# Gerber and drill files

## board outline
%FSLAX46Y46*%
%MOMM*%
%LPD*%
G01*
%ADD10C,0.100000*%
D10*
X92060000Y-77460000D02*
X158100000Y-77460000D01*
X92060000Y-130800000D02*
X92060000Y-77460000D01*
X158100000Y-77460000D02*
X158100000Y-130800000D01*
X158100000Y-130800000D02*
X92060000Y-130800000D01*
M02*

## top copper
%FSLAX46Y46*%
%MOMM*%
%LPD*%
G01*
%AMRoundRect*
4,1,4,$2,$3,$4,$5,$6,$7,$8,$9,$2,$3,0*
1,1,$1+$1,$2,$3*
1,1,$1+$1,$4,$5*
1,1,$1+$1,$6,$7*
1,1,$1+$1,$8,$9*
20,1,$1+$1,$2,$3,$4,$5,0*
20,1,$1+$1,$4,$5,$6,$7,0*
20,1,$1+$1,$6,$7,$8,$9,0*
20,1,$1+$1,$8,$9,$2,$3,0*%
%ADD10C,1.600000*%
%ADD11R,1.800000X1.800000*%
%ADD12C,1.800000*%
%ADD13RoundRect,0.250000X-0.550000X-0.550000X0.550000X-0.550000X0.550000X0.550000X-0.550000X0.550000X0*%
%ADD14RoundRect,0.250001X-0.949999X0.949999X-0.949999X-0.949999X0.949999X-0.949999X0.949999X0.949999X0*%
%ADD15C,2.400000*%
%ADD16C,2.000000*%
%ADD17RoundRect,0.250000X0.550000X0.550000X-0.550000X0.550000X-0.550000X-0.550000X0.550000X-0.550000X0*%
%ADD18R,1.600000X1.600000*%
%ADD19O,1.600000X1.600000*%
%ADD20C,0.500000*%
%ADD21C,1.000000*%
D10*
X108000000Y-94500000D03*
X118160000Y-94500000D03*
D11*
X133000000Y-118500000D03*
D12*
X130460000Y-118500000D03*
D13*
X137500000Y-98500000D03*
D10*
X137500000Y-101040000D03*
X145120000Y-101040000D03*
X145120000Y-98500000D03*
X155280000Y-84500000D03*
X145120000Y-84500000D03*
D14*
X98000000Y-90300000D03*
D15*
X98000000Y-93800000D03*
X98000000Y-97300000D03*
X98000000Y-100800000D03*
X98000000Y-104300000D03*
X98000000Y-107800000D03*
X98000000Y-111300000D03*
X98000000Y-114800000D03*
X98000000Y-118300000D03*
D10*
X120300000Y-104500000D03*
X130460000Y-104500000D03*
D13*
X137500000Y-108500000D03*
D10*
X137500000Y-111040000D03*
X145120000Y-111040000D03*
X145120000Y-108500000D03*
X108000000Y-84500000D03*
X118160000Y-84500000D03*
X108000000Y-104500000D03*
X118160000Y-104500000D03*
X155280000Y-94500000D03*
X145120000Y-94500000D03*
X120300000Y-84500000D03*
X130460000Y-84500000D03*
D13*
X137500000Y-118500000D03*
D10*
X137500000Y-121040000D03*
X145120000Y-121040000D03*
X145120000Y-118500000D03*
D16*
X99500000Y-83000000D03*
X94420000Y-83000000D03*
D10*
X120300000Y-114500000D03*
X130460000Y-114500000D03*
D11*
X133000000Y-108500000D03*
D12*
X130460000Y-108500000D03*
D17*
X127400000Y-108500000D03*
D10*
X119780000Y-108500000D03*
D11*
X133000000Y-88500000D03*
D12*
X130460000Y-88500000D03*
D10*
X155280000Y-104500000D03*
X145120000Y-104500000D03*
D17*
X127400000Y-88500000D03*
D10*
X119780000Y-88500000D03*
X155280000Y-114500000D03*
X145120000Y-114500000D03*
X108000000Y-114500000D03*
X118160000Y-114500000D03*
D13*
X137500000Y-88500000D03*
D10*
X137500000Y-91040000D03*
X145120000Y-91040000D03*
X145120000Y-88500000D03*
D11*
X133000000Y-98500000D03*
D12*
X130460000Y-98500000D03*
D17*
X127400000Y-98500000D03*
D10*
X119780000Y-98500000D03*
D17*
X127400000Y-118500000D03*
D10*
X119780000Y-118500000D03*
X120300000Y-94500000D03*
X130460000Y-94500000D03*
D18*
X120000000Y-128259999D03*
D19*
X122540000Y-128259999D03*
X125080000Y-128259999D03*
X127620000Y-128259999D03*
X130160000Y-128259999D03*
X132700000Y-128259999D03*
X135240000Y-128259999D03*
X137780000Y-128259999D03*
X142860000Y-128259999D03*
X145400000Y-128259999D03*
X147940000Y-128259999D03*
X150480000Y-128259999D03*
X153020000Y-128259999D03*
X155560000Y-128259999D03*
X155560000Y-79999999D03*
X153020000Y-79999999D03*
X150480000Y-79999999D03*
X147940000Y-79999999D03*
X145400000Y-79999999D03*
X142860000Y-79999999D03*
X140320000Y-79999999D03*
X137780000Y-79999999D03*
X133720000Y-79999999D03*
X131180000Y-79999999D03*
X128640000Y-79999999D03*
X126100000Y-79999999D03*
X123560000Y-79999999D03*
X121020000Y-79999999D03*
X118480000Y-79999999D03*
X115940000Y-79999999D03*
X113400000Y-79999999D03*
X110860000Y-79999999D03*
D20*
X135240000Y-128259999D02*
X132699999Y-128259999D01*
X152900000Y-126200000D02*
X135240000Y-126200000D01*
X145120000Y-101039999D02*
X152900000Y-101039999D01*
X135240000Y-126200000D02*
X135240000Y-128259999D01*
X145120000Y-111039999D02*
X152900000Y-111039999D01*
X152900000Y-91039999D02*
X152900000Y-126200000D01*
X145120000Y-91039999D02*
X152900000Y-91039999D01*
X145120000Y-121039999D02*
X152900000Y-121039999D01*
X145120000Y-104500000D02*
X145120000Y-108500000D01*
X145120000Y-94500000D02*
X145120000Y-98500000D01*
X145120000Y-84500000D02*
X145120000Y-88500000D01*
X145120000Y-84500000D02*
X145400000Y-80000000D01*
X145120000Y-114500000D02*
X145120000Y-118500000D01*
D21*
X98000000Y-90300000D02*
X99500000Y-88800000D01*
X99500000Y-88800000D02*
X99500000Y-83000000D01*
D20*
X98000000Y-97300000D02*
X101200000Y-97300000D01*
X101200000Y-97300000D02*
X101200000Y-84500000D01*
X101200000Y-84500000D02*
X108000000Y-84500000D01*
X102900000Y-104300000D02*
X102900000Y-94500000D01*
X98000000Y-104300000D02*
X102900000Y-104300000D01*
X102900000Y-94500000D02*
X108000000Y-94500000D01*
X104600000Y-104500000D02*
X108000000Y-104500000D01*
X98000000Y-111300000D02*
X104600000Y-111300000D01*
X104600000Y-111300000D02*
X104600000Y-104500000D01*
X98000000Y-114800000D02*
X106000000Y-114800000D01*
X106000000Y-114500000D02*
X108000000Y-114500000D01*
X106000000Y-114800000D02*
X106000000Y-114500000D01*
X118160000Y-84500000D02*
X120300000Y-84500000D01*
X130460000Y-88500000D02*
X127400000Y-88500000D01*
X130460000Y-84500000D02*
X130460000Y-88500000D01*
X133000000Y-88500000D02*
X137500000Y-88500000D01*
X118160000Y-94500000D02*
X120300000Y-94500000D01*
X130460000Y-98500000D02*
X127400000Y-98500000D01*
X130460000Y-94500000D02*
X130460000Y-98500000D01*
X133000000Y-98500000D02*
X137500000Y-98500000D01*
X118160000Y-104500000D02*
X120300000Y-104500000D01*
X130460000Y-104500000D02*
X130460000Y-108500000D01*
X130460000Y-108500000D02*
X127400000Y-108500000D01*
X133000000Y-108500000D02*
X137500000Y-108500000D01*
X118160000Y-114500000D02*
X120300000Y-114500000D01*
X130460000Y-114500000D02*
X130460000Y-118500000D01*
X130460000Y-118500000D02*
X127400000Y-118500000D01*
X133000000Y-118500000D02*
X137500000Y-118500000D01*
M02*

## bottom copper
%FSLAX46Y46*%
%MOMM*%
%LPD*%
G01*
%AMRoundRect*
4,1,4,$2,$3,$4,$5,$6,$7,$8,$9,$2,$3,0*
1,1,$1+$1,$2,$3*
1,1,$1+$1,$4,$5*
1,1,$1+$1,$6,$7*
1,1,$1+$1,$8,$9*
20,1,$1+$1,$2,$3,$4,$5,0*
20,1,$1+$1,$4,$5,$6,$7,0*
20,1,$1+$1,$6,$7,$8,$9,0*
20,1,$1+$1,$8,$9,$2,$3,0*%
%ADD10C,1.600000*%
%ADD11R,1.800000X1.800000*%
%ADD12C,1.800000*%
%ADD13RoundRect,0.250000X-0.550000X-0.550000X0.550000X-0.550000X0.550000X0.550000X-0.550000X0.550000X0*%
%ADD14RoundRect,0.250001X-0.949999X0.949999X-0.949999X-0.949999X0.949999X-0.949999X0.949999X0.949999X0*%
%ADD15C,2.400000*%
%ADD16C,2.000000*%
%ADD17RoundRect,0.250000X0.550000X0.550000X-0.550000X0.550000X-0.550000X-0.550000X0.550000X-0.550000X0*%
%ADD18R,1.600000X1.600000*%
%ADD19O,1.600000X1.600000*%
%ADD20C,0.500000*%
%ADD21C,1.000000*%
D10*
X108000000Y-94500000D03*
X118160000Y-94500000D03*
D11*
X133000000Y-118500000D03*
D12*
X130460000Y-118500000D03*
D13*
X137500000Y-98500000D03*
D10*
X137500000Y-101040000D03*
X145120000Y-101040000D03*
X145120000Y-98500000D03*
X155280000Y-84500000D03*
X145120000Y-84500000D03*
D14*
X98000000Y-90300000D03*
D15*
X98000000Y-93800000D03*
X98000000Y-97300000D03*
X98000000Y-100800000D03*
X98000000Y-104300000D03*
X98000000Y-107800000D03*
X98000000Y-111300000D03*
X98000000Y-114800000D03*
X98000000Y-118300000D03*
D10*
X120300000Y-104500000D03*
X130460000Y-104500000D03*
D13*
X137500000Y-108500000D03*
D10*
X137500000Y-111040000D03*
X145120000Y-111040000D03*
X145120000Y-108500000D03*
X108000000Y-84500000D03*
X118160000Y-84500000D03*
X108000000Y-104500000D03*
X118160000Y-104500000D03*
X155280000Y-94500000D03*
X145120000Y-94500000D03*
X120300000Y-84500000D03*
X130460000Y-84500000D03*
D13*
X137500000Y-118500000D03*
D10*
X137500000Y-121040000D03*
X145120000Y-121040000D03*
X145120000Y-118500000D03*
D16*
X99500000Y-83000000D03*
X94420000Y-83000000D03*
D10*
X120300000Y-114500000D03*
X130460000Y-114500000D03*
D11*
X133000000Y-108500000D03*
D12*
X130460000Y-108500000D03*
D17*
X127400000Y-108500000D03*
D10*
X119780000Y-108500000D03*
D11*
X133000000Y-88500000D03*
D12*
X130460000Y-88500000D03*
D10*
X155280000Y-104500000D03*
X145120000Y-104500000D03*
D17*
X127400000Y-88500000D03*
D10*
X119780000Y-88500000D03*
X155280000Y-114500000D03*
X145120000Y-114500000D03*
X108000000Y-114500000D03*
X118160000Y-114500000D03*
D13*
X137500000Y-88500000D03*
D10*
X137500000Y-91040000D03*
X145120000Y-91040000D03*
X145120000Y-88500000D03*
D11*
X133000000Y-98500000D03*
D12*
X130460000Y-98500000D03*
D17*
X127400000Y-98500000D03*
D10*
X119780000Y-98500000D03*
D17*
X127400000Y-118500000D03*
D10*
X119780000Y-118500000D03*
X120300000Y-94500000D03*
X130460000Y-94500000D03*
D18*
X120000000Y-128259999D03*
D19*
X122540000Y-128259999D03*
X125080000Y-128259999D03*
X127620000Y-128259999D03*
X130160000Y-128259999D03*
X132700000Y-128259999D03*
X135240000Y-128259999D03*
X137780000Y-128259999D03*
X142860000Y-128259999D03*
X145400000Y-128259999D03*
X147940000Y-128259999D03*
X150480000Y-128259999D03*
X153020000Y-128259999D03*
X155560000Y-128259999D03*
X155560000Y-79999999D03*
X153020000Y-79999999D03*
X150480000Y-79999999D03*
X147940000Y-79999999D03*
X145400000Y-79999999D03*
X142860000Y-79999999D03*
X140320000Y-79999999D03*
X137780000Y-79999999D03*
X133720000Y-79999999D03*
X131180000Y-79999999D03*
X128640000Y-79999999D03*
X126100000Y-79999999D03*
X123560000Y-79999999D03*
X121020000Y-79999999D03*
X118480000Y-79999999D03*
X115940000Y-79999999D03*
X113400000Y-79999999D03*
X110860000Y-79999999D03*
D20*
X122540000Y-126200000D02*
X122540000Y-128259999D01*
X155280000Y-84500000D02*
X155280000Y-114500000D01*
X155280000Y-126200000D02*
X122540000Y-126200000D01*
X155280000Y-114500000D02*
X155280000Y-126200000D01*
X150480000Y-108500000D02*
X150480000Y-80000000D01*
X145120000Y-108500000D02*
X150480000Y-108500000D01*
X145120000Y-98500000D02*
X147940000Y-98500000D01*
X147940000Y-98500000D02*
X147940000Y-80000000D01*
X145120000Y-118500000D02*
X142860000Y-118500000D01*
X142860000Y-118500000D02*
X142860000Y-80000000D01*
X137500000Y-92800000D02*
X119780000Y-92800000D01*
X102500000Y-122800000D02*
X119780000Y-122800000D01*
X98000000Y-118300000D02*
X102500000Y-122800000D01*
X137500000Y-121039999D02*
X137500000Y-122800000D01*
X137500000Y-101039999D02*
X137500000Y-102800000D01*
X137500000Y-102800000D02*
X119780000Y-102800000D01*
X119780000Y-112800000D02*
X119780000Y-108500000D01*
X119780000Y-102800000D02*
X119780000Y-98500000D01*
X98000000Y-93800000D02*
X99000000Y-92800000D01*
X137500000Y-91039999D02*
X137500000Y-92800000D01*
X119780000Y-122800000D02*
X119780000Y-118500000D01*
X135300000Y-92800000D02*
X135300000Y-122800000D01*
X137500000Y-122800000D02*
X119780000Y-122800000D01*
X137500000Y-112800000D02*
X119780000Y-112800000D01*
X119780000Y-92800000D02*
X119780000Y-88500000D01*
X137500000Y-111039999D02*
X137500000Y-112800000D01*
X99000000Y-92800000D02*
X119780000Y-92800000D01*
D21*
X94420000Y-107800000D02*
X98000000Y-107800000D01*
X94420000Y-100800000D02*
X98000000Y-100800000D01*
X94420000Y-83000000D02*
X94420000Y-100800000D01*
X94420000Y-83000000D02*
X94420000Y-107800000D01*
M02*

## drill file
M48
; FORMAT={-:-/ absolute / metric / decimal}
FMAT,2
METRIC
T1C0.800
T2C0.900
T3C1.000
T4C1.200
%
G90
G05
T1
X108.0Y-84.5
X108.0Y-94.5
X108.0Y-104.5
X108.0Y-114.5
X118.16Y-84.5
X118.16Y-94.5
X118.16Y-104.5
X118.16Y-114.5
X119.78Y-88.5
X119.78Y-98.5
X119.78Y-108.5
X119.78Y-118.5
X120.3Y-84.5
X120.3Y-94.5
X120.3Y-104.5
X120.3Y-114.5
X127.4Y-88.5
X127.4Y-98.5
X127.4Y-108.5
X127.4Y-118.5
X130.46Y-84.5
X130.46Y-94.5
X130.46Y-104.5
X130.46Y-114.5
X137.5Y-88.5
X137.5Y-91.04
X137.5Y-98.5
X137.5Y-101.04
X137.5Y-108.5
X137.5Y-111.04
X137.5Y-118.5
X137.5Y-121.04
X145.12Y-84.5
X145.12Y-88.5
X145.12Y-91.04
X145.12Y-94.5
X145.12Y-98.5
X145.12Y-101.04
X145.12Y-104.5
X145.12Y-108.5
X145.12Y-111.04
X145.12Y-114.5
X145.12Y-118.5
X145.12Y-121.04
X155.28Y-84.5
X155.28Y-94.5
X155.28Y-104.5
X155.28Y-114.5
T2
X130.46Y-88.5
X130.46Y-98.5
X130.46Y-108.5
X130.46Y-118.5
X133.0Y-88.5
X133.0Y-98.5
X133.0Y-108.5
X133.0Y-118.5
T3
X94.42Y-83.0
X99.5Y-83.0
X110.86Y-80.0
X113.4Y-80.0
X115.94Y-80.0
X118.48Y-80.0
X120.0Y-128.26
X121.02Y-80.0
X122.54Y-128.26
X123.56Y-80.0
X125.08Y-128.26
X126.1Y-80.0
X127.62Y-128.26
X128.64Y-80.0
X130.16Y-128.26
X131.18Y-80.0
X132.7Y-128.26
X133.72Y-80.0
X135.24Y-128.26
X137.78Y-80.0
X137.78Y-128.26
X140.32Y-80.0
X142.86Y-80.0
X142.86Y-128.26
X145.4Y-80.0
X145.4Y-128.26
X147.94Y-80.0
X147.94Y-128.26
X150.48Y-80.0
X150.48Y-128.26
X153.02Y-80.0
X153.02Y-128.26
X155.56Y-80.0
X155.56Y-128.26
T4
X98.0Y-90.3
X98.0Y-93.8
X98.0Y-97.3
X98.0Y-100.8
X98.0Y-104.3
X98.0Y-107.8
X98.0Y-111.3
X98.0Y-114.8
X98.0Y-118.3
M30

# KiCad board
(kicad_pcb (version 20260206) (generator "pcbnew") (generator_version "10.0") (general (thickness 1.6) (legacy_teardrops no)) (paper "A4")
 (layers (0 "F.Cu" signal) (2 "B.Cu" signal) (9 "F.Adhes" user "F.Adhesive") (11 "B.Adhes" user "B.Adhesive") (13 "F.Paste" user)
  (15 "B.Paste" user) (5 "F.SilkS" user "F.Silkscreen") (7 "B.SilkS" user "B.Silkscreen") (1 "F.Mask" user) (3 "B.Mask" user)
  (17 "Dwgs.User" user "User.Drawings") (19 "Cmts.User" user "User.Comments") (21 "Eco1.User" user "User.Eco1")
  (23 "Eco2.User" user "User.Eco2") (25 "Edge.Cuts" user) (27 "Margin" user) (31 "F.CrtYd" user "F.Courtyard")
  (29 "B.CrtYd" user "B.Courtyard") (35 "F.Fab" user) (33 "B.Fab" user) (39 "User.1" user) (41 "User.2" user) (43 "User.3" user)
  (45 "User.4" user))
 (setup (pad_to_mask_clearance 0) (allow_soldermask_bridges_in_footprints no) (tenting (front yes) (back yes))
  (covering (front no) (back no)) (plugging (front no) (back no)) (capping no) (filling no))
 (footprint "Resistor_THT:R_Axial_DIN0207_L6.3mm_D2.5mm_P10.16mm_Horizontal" (layer "F.Cu") (at 108 94.5)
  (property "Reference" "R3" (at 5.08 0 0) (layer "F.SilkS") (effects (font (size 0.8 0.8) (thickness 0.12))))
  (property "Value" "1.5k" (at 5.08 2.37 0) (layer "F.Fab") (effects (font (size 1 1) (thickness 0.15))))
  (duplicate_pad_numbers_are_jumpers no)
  (pad "1" thru_hole circle (at 0 0) (size 1.6 1.6) (drill 0.8) (layers "*.Cu" "*.Mask") (remove_unused_layers no) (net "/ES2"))
  (pad "2" thru_hole circle (at 10.16 0) (size 1.6 1.6) (drill 0.8) (layers "*.Cu" "*.Mask") (remove_unused_layers no) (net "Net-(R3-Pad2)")))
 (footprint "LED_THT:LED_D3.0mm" (layer "F.Cu") (at 133 118.5 180)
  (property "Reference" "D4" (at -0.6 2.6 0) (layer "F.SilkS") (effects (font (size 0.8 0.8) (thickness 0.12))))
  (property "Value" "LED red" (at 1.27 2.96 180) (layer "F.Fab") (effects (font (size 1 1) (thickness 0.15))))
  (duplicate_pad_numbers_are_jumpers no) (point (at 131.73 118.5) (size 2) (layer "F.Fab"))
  (pad "1" thru_hole rect (at 0 0 180) (size 1.8 1.8) (drill 0.9) (layers "*.Cu" "*.Mask") (remove_unused_layers no) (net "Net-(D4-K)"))
  (pad "2" thru_hole circle (at 2.54 0 180) (size 1.8 1.8) (drill 0.9) (layers "*.Cu" "*.Mask") (remove_unused_layers no) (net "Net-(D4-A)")))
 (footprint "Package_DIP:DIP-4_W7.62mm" (layer "F.Cu") (at 137.5 98.5)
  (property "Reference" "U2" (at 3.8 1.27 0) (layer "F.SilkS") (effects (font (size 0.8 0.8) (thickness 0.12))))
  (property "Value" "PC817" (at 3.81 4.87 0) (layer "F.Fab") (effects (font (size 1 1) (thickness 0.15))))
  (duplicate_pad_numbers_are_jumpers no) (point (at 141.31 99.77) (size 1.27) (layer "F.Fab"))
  (pad "1" thru_hole roundrect (at 0 0) (size 1.6 1.6) (drill 0.8) (layers "*.Cu" "*.Mask") (remove_unused_layers no)
   (roundrect_rratio 0.15625) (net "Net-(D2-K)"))
  (pad "2" thru_hole circle (at 0 2.54) (size 1.6 1.6) (drill 0.8) (layers "*.Cu" "*.Mask") (remove_unused_layers no) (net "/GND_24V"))
  (pad "3" thru_hole circle (at 7.62 2.54) (size 1.6 1.6) (drill 0.8) (layers "*.Cu" "*.Mask") (remove_unused_layers no) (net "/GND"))
  (pad "4" thru_hole circle (at 7.62 0) (size 1.6 1.6) (drill 0.8) (layers "*.Cu" "*.Mask") (remove_unused_layers no) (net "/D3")))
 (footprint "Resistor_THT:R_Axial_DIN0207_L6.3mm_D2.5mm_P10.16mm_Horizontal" (layer "F.Cu") (at 155.28 84.5 180)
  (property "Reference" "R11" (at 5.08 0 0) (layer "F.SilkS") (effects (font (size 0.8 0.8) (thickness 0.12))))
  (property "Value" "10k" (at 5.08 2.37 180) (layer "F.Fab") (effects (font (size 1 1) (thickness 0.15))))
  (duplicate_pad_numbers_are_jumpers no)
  (pad "1" thru_hole circle (at 0 0 180) (size 1.6 1.6) (drill 0.8) (layers "*.Cu" "*.Mask") (remove_unused_layers no) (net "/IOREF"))
  (pad "2" thru_hole circle (at 10.16 0 180) (size 1.6 1.6) (drill 0.8) (layers "*.Cu" "*.Mask") (remove_unused_layers no) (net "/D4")))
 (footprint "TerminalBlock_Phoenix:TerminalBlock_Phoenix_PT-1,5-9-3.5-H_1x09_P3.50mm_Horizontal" (layer "F.Cu") (at 98 90.3 -90)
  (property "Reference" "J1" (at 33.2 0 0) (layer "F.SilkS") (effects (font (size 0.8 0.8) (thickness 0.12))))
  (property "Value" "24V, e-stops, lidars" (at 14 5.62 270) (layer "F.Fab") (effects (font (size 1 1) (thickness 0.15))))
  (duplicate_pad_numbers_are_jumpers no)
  (pad "1" thru_hole roundrect (at 0 0 270) (size 2.4 2.4) (drill 1.2) (layers "*.Cu" "*.Mask") (remove_unused_layers no)
   (roundrect_rratio 0.104167) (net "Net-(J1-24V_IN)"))
  (pad "2" thru_hole circle (at 3.5 0 270) (size 2.4 2.4) (drill 1.2) (layers "*.Cu" "*.Mask") (remove_unused_layers no) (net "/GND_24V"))
  (pad "3" thru_hole circle (at 7 0 270) (size 2.4 2.4) (drill 1.2) (layers "*.Cu" "*.Mask") (remove_unused_layers no) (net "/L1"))
  (pad "4" thru_hole circle (at 10.5 0 270) (size 2.4 2.4) (drill 1.2) (layers "*.Cu" "*.Mask") (remove_unused_layers no) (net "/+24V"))
  (pad "5" thru_hole circle (at 14 0 270) (size 2.4 2.4) (drill 1.2) (layers "*.Cu" "*.Mask") (remove_unused_layers no) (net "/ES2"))
  (pad "6" thru_hole circle (at 17.5 0 270) (size 2.4 2.4) (drill 1.2) (layers "*.Cu" "*.Mask") (remove_unused_layers no) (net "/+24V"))
  (pad "7" thru_hole circle (at 21 0 270) (size 2.4 2.4) (drill 1.2) (layers "*.Cu" "*.Mask") (remove_unused_layers no) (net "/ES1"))
  (pad "8" thru_hole circle (at 24.5 0 270) (size 2.4 2.4) (drill 1.2) (layers "*.Cu" "*.Mask") (remove_unused_layers no) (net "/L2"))
  (pad "9" thru_hole circle (at 28 0 270) (size 2.4 2.4) (drill 1.2) (layers "*.Cu" "*.Mask") (remove_unused_layers no) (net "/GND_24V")))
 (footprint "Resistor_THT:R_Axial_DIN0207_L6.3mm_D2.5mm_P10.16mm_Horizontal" (layer "F.Cu") (at 120.3 104.5)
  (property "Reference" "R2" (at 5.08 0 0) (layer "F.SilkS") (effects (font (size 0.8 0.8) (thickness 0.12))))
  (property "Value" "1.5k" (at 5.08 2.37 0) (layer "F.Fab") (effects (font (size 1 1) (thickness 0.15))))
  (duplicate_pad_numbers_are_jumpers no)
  (pad "1" thru_hole circle (at 0 0) (size 1.6 1.6) (drill 0.8) (layers "*.Cu" "*.Mask") (remove_unused_layers no) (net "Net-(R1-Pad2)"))
  (pad "2" thru_hole circle (at 10.16 0) (size 1.6 1.6) (drill 0.8) (layers "*.Cu" "*.Mask") (remove_unused_layers no) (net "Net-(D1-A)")))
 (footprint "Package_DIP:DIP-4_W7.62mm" (layer "F.Cu") (at 137.5 108.5)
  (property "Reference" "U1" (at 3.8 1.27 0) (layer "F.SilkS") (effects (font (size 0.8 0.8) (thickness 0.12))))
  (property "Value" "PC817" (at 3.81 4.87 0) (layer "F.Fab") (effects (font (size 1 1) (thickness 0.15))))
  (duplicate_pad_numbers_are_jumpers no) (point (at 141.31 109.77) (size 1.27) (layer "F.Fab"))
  (pad "1" thru_hole roundrect (at 0 0) (size 1.6 1.6) (drill 0.8) (layers "*.Cu" "*.Mask") (remove_unused_layers no)
   (roundrect_rratio 0.15625) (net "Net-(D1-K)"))
  (pad "2" thru_hole circle (at 0 2.54) (size 1.6 1.6) (drill 0.8) (layers "*.Cu" "*.Mask") (remove_unused_layers no) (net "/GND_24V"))
  (pad "3" thru_hole circle (at 7.62 2.54) (size 1.6 1.6) (drill 0.8) (layers "*.Cu" "*.Mask") (remove_unused_layers no) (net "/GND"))
  (pad "4" thru_hole circle (at 7.62 0) (size 1.6 1.6) (drill 0.8) (layers "*.Cu" "*.Mask") (remove_unused_layers no) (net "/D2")))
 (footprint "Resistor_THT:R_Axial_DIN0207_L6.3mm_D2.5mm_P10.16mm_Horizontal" (layer "F.Cu") (at 108 84.5)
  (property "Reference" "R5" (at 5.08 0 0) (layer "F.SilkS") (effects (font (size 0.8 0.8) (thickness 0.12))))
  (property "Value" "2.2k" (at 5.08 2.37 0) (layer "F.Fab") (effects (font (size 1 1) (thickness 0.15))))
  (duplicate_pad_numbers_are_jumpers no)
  (pad "1" thru_hole circle (at 0 0) (size 1.6 1.6) (drill 0.8) (layers "*.Cu" "*.Mask") (remove_unused_layers no) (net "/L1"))
  (pad "2" thru_hole circle (at 10.16 0) (size 1.6 1.6) (drill 0.8) (layers "*.Cu" "*.Mask") (remove_unused_layers no) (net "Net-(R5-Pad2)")))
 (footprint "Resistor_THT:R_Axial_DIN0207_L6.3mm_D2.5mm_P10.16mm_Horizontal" (layer "F.Cu") (at 108 104.5)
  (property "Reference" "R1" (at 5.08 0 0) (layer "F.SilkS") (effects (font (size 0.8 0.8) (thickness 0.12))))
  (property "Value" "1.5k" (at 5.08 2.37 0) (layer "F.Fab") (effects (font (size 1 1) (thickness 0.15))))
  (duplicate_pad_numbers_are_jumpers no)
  (pad "1" thru_hole circle (at 0 0) (size 1.6 1.6) (drill 0.8) (layers "*.Cu" "*.Mask") (remove_unused_layers no) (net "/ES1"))
  (pad "2" thru_hole circle (at 10.16 0) (size 1.6 1.6) (drill 0.8) (layers "*.Cu" "*.Mask") (remove_unused_layers no) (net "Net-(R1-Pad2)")))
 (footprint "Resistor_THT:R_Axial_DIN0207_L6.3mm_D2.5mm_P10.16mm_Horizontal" (layer "F.Cu") (at 155.28 94.5 180)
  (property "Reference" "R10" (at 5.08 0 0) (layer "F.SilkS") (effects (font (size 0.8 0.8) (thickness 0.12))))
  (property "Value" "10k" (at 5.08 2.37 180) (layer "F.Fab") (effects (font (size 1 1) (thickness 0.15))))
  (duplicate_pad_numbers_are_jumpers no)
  (pad "1" thru_hole circle (at 0 0 180) (size 1.6 1.6) (drill 0.8) (layers "*.Cu" "*.Mask") (remove_unused_layers no) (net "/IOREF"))
  (pad "2" thru_hole circle (at 10.16 0 180) (size 1.6 1.6) (drill 0.8) (layers "*.Cu" "*.Mask") (remove_unused_layers no) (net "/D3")))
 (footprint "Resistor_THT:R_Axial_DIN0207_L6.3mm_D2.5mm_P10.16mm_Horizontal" (layer "F.Cu") (at 120.3 84.5)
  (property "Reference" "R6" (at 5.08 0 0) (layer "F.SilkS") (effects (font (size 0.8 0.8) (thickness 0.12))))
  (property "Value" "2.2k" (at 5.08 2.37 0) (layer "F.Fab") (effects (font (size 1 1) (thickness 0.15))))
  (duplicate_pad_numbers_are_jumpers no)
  (pad "1" thru_hole circle (at 0 0) (size 1.6 1.6) (drill 0.8) (layers "*.Cu" "*.Mask") (remove_unused_layers no) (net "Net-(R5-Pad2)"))
  (pad "2" thru_hole circle (at 10.16 0) (size 1.6 1.6) (drill 0.8) (layers "*.Cu" "*.Mask") (remove_unused_layers no) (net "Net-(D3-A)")))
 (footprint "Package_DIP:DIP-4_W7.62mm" (layer "F.Cu") (at 137.5 118.5)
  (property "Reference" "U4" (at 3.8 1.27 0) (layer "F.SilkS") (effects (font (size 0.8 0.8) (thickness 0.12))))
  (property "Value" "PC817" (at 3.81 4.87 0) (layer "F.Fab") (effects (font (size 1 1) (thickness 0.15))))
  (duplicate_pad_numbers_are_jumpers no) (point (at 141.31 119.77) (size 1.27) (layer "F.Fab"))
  (pad "1" thru_hole roundrect (at 0 0) (size 1.6 1.6) (drill 0.8) (layers "*.Cu" "*.Mask") (remove_unused_layers no)
   (roundrect_rratio 0.15625) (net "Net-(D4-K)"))
  (pad "2" thru_hole circle (at 0 2.54) (size 1.6 1.6) (drill 0.8) (layers "*.Cu" "*.Mask") (remove_unused_layers no) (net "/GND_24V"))
  (pad "3" thru_hole circle (at 7.62 2.54) (size 1.6 1.6) (drill 0.8) (layers "*.Cu" "*.Mask") (remove_unused_layers no) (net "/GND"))
  (pad "4" thru_hole circle (at 7.62 0) (size 1.6 1.6) (drill 0.8) (layers "*.Cu" "*.Mask") (remove_unused_layers no) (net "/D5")))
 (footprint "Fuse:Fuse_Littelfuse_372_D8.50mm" (layer "F.Cu") (at 99.5 83 180)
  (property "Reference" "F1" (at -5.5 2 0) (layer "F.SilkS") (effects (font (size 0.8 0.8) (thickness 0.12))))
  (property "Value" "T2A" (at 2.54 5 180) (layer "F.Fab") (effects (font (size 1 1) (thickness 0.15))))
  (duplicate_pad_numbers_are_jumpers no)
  (pad "1" thru_hole circle (at 0 0 180) (size 2 2) (drill 1) (layers "*.Cu" "*.Mask") (remove_unused_layers no) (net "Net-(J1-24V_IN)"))
  (pad "2" thru_hole circle (at 5.08 0 180) (size 2 2) (drill 1) (layers "*.Cu" "*.Mask") (remove_unused_layers no) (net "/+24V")))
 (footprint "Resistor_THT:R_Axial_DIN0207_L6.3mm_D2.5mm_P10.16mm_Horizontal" (layer "F.Cu") (at 120.3 114.5)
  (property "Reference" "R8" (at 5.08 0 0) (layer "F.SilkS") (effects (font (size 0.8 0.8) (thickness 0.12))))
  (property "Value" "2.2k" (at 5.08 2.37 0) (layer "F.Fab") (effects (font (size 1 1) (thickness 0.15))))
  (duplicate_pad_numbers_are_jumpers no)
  (pad "1" thru_hole circle (at 0 0) (size 1.6 1.6) (drill 0.8) (layers "*.Cu" "*.Mask") (remove_unused_layers no) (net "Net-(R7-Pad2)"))
  (pad "2" thru_hole circle (at 10.16 0) (size 1.6 1.6) (drill 0.8) (layers "*.Cu" "*.Mask") (remove_unused_layers no) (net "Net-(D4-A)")))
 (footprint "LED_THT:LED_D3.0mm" (layer "F.Cu") (at 133 108.5 180)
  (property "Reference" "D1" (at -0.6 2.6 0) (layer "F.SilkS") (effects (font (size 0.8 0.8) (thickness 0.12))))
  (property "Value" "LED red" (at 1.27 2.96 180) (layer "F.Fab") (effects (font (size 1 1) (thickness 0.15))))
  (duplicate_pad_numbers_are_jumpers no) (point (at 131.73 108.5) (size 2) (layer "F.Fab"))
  (pad "1" thru_hole rect (at 0 0 180) (size 1.8 1.8) (drill 0.9) (layers "*.Cu" "*.Mask") (remove_unused_layers no) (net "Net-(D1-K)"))
  (pad "2" thru_hole circle (at 2.54 0 180) (size 1.8 1.8) (drill 0.9) (layers "*.Cu" "*.Mask") (remove_unused_layers no) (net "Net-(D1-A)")))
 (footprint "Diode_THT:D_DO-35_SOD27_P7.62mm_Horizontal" (layer "F.Cu") (at 127.4 108.5 180)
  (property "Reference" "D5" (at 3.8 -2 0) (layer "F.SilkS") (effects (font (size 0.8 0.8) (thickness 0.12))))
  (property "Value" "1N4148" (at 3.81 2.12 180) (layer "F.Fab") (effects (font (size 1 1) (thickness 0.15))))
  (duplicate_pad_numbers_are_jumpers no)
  (pad "1" thru_hole roundrect (at 0 0 180) (size 1.6 1.6) (drill 0.8) (layers "*.Cu" "*.Mask") (remove_unused_layers no)
   (roundrect_rratio 0.15625) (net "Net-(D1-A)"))
  (pad "2" thru_hole circle (at 7.62 0 180) (size 1.6 1.6) (drill 0.8) (layers "*.Cu" "*.Mask") (remove_unused_layers no) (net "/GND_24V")))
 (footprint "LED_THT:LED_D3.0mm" (layer "F.Cu") (at 133 88.5 180)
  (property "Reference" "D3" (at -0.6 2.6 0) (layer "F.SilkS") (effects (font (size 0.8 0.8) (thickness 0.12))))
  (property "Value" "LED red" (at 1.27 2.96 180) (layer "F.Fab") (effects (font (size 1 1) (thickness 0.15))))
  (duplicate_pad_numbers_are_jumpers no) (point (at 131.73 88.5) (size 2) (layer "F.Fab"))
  (pad "1" thru_hole rect (at 0 0 180) (size 1.8 1.8) (drill 0.9) (layers "*.Cu" "*.Mask") (remove_unused_layers no) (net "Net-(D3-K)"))
  (pad "2" thru_hole circle (at 2.54 0 180) (size 1.8 1.8) (drill 0.9) (layers "*.Cu" "*.Mask") (remove_unused_layers no) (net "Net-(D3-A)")))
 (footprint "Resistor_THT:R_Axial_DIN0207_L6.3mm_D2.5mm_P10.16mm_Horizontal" (layer "F.Cu") (at 155.28 104.5 180)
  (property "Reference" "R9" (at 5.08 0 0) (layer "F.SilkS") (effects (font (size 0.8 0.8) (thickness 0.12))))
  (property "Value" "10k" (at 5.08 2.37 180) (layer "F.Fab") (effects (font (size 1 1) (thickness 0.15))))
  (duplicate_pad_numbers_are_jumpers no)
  (pad "1" thru_hole circle (at 0 0 180) (size 1.6 1.6) (drill 0.8) (layers "*.Cu" "*.Mask") (remove_unused_layers no) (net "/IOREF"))
  (pad "2" thru_hole circle (at 10.16 0 180) (size 1.6 1.6) (drill 0.8) (layers "*.Cu" "*.Mask") (remove_unused_layers no) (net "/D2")))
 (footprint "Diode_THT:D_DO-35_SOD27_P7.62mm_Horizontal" (layer "F.Cu") (at 127.4 88.5 180)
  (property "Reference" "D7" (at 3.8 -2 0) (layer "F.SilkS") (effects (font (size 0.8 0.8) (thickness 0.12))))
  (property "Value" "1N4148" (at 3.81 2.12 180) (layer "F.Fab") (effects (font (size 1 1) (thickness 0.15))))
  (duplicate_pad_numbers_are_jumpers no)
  (pad "1" thru_hole roundrect (at 0 0 180) (size 1.6 1.6) (drill 0.8) (layers "*.Cu" "*.Mask") (remove_unused_layers no)
   (roundrect_rratio 0.15625) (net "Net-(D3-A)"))
  (pad "2" thru_hole circle (at 7.62 0 180) (size 1.6 1.6) (drill 0.8) (layers "*.Cu" "*.Mask") (remove_unused_layers no) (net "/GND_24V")))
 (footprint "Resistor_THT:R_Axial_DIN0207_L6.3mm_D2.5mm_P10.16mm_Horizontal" (layer "F.Cu") (at 155.28 114.5 180)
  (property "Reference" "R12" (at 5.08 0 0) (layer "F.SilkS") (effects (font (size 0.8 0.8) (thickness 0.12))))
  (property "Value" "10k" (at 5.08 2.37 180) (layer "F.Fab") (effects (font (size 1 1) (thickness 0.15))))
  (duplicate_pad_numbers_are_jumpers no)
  (pad "1" thru_hole circle (at 0 0 180) (size 1.6 1.6) (drill 0.8) (layers "*.Cu" "*.Mask") (remove_unused_layers no) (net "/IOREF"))
  (pad "2" thru_hole circle (at 10.16 0 180) (size 1.6 1.6) (drill 0.8) (layers "*.Cu" "*.Mask") (remove_unused_layers no) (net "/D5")))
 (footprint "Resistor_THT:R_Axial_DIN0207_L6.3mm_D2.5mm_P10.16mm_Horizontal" (layer "F.Cu") (at 108 114.5)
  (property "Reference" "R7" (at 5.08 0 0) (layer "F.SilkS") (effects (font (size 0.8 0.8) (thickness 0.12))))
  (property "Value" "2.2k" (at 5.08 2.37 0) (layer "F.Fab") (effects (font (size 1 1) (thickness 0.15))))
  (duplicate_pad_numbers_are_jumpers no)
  (pad "1" thru_hole circle (at 0 0) (size 1.6 1.6) (drill 0.8) (layers "*.Cu" "*.Mask") (remove_unused_layers no) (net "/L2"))
  (pad "2" thru_hole circle (at 10.16 0) (size 1.6 1.6) (drill 0.8) (layers "*.Cu" "*.Mask") (remove_unused_layers no) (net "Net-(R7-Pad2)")))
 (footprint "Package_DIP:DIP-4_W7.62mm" (layer "F.Cu") (at 137.5 88.5)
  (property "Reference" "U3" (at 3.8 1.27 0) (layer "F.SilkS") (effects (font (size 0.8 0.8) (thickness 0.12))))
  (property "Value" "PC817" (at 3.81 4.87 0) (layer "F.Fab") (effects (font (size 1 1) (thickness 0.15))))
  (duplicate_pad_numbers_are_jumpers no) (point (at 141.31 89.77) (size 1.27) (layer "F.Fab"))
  (pad "1" thru_hole roundrect (at 0 0) (size 1.6 1.6) (drill 0.8) (layers "*.Cu" "*.Mask") (remove_unused_layers no)
   (roundrect_rratio 0.15625) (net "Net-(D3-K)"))
  (pad "2" thru_hole circle (at 0 2.54) (size 1.6 1.6) (drill 0.8) (layers "*.Cu" "*.Mask") (remove_unused_layers no) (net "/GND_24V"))
  (pad "3" thru_hole circle (at 7.62 2.54) (size 1.6 1.6) (drill 0.8) (layers "*.Cu" "*.Mask") (remove_unused_layers no) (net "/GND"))
  (pad "4" thru_hole circle (at 7.62 0) (size 1.6 1.6) (drill 0.8) (layers "*.Cu" "*.Mask") (remove_unused_layers no) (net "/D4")))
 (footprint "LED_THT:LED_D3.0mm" (layer "F.Cu") (at 133 98.5 180)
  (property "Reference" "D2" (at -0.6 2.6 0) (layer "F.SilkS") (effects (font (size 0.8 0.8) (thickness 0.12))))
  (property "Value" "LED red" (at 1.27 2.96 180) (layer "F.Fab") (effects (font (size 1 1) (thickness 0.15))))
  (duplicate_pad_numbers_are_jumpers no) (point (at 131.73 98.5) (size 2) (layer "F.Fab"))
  (pad "1" thru_hole rect (at 0 0 180) (size 1.8 1.8) (drill 0.9) (layers "*.Cu" "*.Mask") (remove_unused_layers no) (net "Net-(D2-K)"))
  (pad "2" thru_hole circle (at 2.54 0 180) (size 1.8 1.8) (drill 0.9) (layers "*.Cu" "*.Mask") (remove_unused_layers no) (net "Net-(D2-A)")))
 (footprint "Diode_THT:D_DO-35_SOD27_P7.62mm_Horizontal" (layer "F.Cu") (at 127.4 98.5 180)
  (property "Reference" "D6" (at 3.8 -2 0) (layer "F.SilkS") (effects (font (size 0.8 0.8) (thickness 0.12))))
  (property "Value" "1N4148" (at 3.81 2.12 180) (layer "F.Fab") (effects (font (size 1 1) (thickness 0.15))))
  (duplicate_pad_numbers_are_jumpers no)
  (pad "1" thru_hole roundrect (at 0 0 180) (size 1.6 1.6) (drill 0.8) (layers "*.Cu" "*.Mask") (remove_unused_layers no)
   (roundrect_rratio 0.15625) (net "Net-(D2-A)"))
  (pad "2" thru_hole circle (at 7.62 0 180) (size 1.6 1.6) (drill 0.8) (layers "*.Cu" "*.Mask") (remove_unused_layers no) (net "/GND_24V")))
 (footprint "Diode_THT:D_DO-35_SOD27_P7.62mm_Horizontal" (layer "F.Cu") (at 127.4 118.5 180)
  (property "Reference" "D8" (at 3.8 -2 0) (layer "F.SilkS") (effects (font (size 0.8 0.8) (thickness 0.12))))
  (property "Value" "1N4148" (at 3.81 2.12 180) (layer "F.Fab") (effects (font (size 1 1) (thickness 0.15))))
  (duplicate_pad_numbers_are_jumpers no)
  (pad "1" thru_hole roundrect (at 0 0 180) (size 1.6 1.6) (drill 0.8) (layers "*.Cu" "*.Mask") (remove_unused_layers no)
   (roundrect_rratio 0.15625) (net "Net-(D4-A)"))
  (pad "2" thru_hole circle (at 7.62 0 180) (size 1.6 1.6) (drill 0.8) (layers "*.Cu" "*.Mask") (remove_unused_layers no) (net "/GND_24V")))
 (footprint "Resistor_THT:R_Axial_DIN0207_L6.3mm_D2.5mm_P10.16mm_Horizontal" (layer "F.Cu") (at 120.3 94.5)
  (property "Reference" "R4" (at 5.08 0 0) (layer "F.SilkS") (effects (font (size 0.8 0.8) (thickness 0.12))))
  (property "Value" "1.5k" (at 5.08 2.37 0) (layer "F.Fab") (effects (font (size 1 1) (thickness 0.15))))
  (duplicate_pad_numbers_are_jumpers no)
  (pad "1" thru_hole circle (at 0 0) (size 1.6 1.6) (drill 0.8) (layers "*.Cu" "*.Mask") (remove_unused_layers no) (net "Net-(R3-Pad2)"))
  (pad "2" thru_hole circle (at 10.16 0) (size 1.6 1.6) (drill 0.8) (layers "*.Cu" "*.Mask") (remove_unused_layers no) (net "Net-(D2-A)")))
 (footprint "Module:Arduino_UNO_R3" (layer "B.Cu") (at 120 128.259999)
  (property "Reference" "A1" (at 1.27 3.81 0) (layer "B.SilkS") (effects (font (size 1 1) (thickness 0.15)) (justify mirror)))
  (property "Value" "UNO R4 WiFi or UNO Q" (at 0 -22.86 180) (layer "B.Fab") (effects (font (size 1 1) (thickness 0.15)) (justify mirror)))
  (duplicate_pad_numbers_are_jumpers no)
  (pad "1" thru_hole rect (at 0 0 270) (size 1.6 1.6) (drill 1) (layers "*.Cu" "*.Mask") (remove_unused_layers no)
   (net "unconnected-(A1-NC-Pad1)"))
  (pad "2" thru_hole oval (at 2.54 0 270) (size 1.6 1.6) (drill 1) (layers "*.Cu" "*.Mask") (remove_unused_layers no) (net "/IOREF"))
  (pad "3" thru_hole oval (at 5.08 0 270) (size 1.6 1.6) (drill 1) (layers "*.Cu" "*.Mask") (remove_unused_layers no)
   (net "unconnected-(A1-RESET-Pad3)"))
  (pad "4" thru_hole oval (at 7.62 0 270) (size 1.6 1.6) (drill 1) (layers "*.Cu" "*.Mask") (remove_unused_layers no)
   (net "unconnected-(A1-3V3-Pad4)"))
  (pad "5" thru_hole oval (at 10.16 0 270) (size 1.6 1.6) (drill 1) (layers "*.Cu" "*.Mask") (remove_unused_layers no)
   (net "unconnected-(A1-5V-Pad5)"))
  (pad "6" thru_hole oval (at 12.7 0 270) (size 1.6 1.6) (drill 1) (layers "*.Cu" "*.Mask") (remove_unused_layers no) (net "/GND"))
  (pad "7" thru_hole oval (at 15.24 0 270) (size 1.6 1.6) (drill 1) (layers "*.Cu" "*.Mask") (remove_unused_layers no) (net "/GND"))
  (pad "8" thru_hole oval (at 17.78 0 270) (size 1.6 1.6) (drill 1) (layers "*.Cu" "*.Mask") (remove_unused_layers no)
   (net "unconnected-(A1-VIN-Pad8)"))
  (pad "9" thru_hole oval (at 22.86 0 270) (size 1.6 1.6) (drill 1) (layers "*.Cu" "*.Mask") (remove_unused_layers no)
   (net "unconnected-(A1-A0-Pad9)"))
  (pad "10" thru_hole oval (at 25.4 0 270) (size 1.6 1.6) (drill 1) (layers "*.Cu" "*.Mask") (remove_unused_layers no)
   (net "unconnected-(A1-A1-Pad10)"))
  (pad "11" thru_hole oval (at 27.94 0 270) (size 1.6 1.6) (drill 1) (layers "*.Cu" "*.Mask") (remove_unused_layers no)
   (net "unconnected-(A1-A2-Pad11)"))
  (pad "12" thru_hole oval (at 30.48 0 270) (size 1.6 1.6) (drill 1) (layers "*.Cu" "*.Mask") (remove_unused_layers no)
   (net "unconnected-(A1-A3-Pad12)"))
  (pad "13" thru_hole oval (at 33.02 0 270) (size 1.6 1.6) (drill 1) (layers "*.Cu" "*.Mask") (remove_unused_layers no)
   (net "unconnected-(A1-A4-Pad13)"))
  (pad "14" thru_hole oval (at 35.56 0 270) (size 1.6 1.6) (drill 1) (layers "*.Cu" "*.Mask") (remove_unused_layers no)
   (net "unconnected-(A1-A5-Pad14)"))
  (pad "15" thru_hole oval (at 35.56 -48.26 270) (size 1.6 1.6) (drill 1) (layers "*.Cu" "*.Mask") (remove_unused_layers no)
   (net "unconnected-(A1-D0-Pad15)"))
  (pad "16" thru_hole oval (at 33.02 -48.26 270) (size 1.6 1.6) (drill 1) (layers "*.Cu" "*.Mask") (remove_unused_layers no)
   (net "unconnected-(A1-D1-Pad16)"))
  (pad "17" thru_hole oval (at 30.48 -48.26 270) (size 1.6 1.6) (drill 1) (layers "*.Cu" "*.Mask") (remove_unused_layers no) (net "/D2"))
  (pad "18" thru_hole oval (at 27.94 -48.26 270) (size 1.6 1.6) (drill 1) (layers "*.Cu" "*.Mask") (remove_unused_layers no) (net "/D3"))
  (pad "19" thru_hole oval (at 25.4 -48.26 270) (size 1.6 1.6) (drill 1) (layers "*.Cu" "*.Mask") (remove_unused_layers no) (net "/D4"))
  (pad "20" thru_hole oval (at 22.86 -48.26 270) (size 1.6 1.6) (drill 1) (layers "*.Cu" "*.Mask") (remove_unused_layers no) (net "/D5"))
  (pad "21" thru_hole oval (at 20.32 -48.26 270) (size 1.6 1.6) (drill 1) (layers "*.Cu" "*.Mask") (remove_unused_layers no)
   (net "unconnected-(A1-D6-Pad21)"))
  (pad "22" thru_hole oval (at 17.78 -48.26 270) (size 1.6 1.6) (drill 1) (layers "*.Cu" "*.Mask") (remove_unused_layers no)
   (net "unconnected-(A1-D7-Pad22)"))
  (pad "23" thru_hole oval (at 13.72 -48.26 270) (size 1.6 1.6) (drill 1) (layers "*.Cu" "*.Mask") (remove_unused_layers no)
   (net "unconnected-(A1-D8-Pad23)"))
  (pad "24" thru_hole oval (at 11.18 -48.26 270) (size 1.6 1.6) (drill 1) (layers "*.Cu" "*.Mask") (remove_unused_layers no)
   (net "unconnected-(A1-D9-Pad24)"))
  (pad "25" thru_hole oval (at 8.64 -48.26 270) (size 1.6 1.6) (drill 1) (layers "*.Cu" "*.Mask") (remove_unused_layers no)
   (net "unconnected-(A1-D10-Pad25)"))
  (pad "26" thru_hole oval (at 6.1 -48.26 270) (size 1.6 1.6) (drill 1) (layers "*.Cu" "*.Mask") (remove_unused_layers no)
   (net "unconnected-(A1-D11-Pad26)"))
  (pad "27" thru_hole oval (at 3.56 -48.26 270) (size 1.6 1.6) (drill 1) (layers "*.Cu" "*.Mask") (remove_unused_layers no)
   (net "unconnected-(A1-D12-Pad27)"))
  (pad "28" thru_hole oval (at 1.02 -48.26 270) (size 1.6 1.6) (drill 1) (layers "*.Cu" "*.Mask") (remove_unused_layers no)
   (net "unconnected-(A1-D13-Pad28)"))
  (pad "29" thru_hole oval (at -1.52 -48.26 270) (size 1.6 1.6) (drill 1) (layers "*.Cu" "*.Mask") (remove_unused_layers no)
   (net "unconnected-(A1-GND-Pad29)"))
  (pad "30" thru_hole oval (at -4.06 -48.26 270) (size 1.6 1.6) (drill 1) (layers "*.Cu" "*.Mask") (remove_unused_layers no)
   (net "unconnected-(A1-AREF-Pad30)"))
  (pad "31" thru_hole oval (at -6.6 -48.26 270) (size 1.6 1.6) (drill 1) (layers "*.Cu" "*.Mask") (remove_unused_layers no)
   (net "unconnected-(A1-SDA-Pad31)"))
  (pad "32" thru_hole oval (at -9.14 -48.26 270) (size 1.6 1.6) (drill 1) (layers "*.Cu" "*.Mask") (remove_unused_layers no)
   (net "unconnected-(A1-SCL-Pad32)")))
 (gr_line (start 92.06 77.46) (end 158.1 77.46) (stroke (width 0.1) (type default)) (layer "Edge.Cuts"))
 (gr_line (start 92.06 130.8) (end 92.06 77.46) (stroke (width 0.1) (type default)) (layer "Edge.Cuts"))
 (gr_line (start 158.1 77.46) (end 158.1 130.8) (stroke (width 0.1) (type default)) (layer "Edge.Cuts"))
 (gr_line (start 158.1 130.8) (end 92.06 130.8) (stroke (width 0.1) (type default)) (layer "Edge.Cuts"))
 (segment (start 122.54 126.2) (end 122.54 128.259999) (width 0.5) (layer "B.Cu") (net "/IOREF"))
 (segment (start 155.28 84.5) (end 155.28 114.5) (width 0.5) (layer "B.Cu") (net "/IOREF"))
 (segment (start 155.28 126.2) (end 122.54 126.2) (width 0.5) (layer "B.Cu") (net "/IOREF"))
 (segment (start 155.28 114.5) (end 155.28 126.2) (width 0.5) (layer "B.Cu") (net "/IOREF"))
 (segment (start 135.24 128.259999) (end 132.699999 128.259999) (width 0.5) (layer "F.Cu") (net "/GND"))
 (segment (start 152.9 126.2) (end 135.24 126.2) (width 0.5) (layer "F.Cu") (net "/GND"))
 (segment (start 145.12 101.039999) (end 152.9 101.039999) (width 0.5) (layer "F.Cu") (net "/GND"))
 (segment (start 135.24 126.2) (end 135.24 128.259999) (width 0.5) (layer "F.Cu") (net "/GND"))
 (segment (start 145.12 111.039999) (end 152.9 111.039999) (width 0.5) (layer "F.Cu") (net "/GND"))
 (segment (start 152.9 91.039999) (end 152.9 126.2) (width 0.5) (layer "F.Cu") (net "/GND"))
 (segment (start 145.12 91.039999) (end 152.9 91.039999) (width 0.5) (layer "F.Cu") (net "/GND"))
 (segment (start 145.12 121.039999) (end 152.9 121.039999) (width 0.5) (layer "F.Cu") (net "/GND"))
 (segment (start 145.12 104.5) (end 145.12 108.5) (width 0.5) (layer "F.Cu") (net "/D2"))
 (segment (start 150.48 108.5) (end 150.48 80) (width 0.5) (layer "B.Cu") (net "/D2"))
 (segment (start 145.12 108.5) (end 150.48 108.5) (width 0.5) (layer "B.Cu") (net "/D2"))
 (segment (start 145.12 94.5) (end 145.12 98.5) (width 0.5) (layer "F.Cu") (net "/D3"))
 (segment (start 145.12 98.5) (end 147.94 98.5) (width 0.5) (layer "B.Cu") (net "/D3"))
 (segment (start 147.94 98.5) (end 147.94 80) (width 0.5) (layer "B.Cu") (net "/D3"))
 (segment (start 145.12 84.5) (end 145.12 88.5) (width 0.5) (layer "F.Cu") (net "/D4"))
 (segment (start 145.12 84.5) (end 145.4 80) (width 0.5) (layer "F.Cu") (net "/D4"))
 (segment (start 145.12 114.5) (end 145.12 118.5) (width 0.5) (layer "F.Cu") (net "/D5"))
 (segment (start 145.12 118.5) (end 142.86 118.5) (width 0.5) (layer "B.Cu") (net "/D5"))
 (segment (start 142.86 118.5) (end 142.86 80) (width 0.5) (layer "B.Cu") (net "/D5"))
 (segment (start 98 90.3) (end 99.5 88.8) (width 1) (layer "F.Cu") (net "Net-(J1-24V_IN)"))
 (segment (start 99.5 88.8) (end 99.5 83) (width 1) (layer "F.Cu") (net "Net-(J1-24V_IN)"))
 (segment (start 137.5 92.8) (end 119.78 92.8) (width 0.5) (layer "B.Cu") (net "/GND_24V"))
 (segment (start 102.5 122.8) (end 119.78 122.8) (width 0.5) (layer "B.Cu") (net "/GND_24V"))
 (segment (start 98 118.3) (end 102.5 122.8) (width 0.5) (layer "B.Cu") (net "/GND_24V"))
 (segment (start 137.5 121.039999) (end 137.5 122.8) (width 0.5) (layer "B.Cu") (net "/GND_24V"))
 (segment (start 137.5 101.039999) (end 137.5 102.8) (width 0.5) (layer "B.Cu") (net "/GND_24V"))
 (segment (start 137.5 102.8) (end 119.78 102.8) (width 0.5) (layer "B.Cu") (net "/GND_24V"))
 (segment (start 119.78 112.8) (end 119.78 108.5) (width 0.5) (layer "B.Cu") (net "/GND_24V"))
 (segment (start 119.78 102.8) (end 119.78 98.5) (width 0.5) (layer "B.Cu") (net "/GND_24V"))
 (segment (start 98 93.8) (end 99 92.8) (width 0.5) (layer "B.Cu") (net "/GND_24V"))
 (segment (start 137.5 91.039999) (end 137.5 92.8) (width 0.5) (layer "B.Cu") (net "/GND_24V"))
 (segment (start 119.78 122.8) (end 119.78 118.5) (width 0.5) (layer "B.Cu") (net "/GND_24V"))
 (segment (start 135.3 92.8) (end 135.3 122.8) (width 0.5) (layer "B.Cu") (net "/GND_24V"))
 (segment (start 137.5 122.8) (end 119.78 122.8) (width 0.5) (layer "B.Cu") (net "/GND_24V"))
 (segment (start 137.5 112.8) (end 119.78 112.8) (width 0.5) (layer "B.Cu") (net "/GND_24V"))
 (segment (start 119.78 92.8) (end 119.78 88.5) (width 0.5) (layer "B.Cu") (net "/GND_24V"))
 (segment (start 137.5 111.039999) (end 137.5 112.8) (width 0.5) (layer "B.Cu") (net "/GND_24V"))
 (segment (start 99 92.8) (end 119.78 92.8) (width 0.5) (layer "B.Cu") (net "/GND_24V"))
 (segment (start 98 97.3) (end 101.2 97.3) (width 0.5) (layer "F.Cu") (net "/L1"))
 (segment (start 101.2 97.3) (end 101.2 84.5) (width 0.5) (layer "F.Cu") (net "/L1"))
 (segment (start 101.2 84.5) (end 108 84.5) (width 0.5) (layer "F.Cu") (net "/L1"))
 (segment (start 94.42 107.8) (end 98 107.8) (width 1) (layer "B.Cu") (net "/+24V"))
 (segment (start 94.42 100.8) (end 98 100.8) (width 1) (layer "B.Cu") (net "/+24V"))
 (segment (start 94.42 83) (end 94.42 100.8) (width 1) (layer "B.Cu") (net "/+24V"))
 (segment (start 94.42 83) (end 94.42 107.8) (width 1) (layer "B.Cu") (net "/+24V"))
 (segment (start 102.9 104.3) (end 102.9 94.5) (width 0.5) (layer "F.Cu") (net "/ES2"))
 (segment (start 98 104.3) (end 102.9 104.3) (width 0.5) (layer "F.Cu") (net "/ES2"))
 (segment (start 102.9 94.5) (end 108 94.5) (width 0.5) (layer "F.Cu") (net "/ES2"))
 (segment (start 104.6 104.5) (end 108 104.5) (width 0.5) (layer "F.Cu") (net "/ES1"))
 (segment (start 98 111.3) (end 104.6 111.3) (width 0.5) (layer "F.Cu") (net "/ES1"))
 (segment (start 104.6 111.3) (end 104.6 104.5) (width 0.5) (layer "F.Cu") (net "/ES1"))
 (segment (start 98 114.8) (end 106 114.8) (width 0.5) (layer "F.Cu") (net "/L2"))
 (segment (start 106 114.5) (end 108 114.5) (width 0.5) (layer "F.Cu") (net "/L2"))
 (segment (start 106 114.8) (end 106 114.5) (width 0.5) (layer "F.Cu") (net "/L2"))
 (segment (start 118.16 84.5) (end 120.3 84.5) (width 0.5) (layer "F.Cu") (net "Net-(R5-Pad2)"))
 (segment (start 130.46 88.5) (end 127.4 88.5) (width 0.5) (layer "F.Cu") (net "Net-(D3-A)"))
 (segment (start 130.46 84.5) (end 130.46 88.5) (width 0.5) (layer "F.Cu") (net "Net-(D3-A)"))
 (segment (start 133 88.5) (end 137.5 88.5) (width 0.5) (layer "F.Cu") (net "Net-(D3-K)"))
 (segment (start 118.16 94.5) (end 120.3 94.5) (width 0.5) (layer "F.Cu") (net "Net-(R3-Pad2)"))
 (segment (start 130.46 98.5) (end 127.4 98.5) (width 0.5) (layer "F.Cu") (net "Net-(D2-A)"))
 (segment (start 130.46 94.5) (end 130.46 98.5) (width 0.5) (layer "F.Cu") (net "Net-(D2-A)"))
 (segment (start 133 98.5) (end 137.5 98.5) (width 0.5) (layer "F.Cu") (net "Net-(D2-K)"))
 (segment (start 118.16 104.5) (end 120.3 104.5) (width 0.5) (layer "F.Cu") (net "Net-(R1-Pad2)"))
 (segment (start 130.46 104.5) (end 130.46 108.5) (width 0.5) (layer "F.Cu") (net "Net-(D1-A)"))
 (segment (start 130.46 108.5) (end 127.4 108.5) (width 0.5) (layer "F.Cu") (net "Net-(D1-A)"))
 (segment (start 133 108.5) (end 137.5 108.5) (width 0.5) (layer "F.Cu") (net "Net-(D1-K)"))
 (segment (start 118.16 114.5) (end 120.3 114.5) (width 0.5) (layer "F.Cu") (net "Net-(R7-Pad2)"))
 (segment (start 130.46 114.5) (end 130.46 118.5) (width 0.5) (layer "F.Cu") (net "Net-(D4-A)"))
 (segment (start 130.46 118.5) (end 127.4 118.5) (width 0.5) (layer "F.Cu") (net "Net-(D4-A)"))
 (segment (start 133 118.5) (end 137.5 118.5) (width 0.5) (layer "F.Cu") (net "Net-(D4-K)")))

